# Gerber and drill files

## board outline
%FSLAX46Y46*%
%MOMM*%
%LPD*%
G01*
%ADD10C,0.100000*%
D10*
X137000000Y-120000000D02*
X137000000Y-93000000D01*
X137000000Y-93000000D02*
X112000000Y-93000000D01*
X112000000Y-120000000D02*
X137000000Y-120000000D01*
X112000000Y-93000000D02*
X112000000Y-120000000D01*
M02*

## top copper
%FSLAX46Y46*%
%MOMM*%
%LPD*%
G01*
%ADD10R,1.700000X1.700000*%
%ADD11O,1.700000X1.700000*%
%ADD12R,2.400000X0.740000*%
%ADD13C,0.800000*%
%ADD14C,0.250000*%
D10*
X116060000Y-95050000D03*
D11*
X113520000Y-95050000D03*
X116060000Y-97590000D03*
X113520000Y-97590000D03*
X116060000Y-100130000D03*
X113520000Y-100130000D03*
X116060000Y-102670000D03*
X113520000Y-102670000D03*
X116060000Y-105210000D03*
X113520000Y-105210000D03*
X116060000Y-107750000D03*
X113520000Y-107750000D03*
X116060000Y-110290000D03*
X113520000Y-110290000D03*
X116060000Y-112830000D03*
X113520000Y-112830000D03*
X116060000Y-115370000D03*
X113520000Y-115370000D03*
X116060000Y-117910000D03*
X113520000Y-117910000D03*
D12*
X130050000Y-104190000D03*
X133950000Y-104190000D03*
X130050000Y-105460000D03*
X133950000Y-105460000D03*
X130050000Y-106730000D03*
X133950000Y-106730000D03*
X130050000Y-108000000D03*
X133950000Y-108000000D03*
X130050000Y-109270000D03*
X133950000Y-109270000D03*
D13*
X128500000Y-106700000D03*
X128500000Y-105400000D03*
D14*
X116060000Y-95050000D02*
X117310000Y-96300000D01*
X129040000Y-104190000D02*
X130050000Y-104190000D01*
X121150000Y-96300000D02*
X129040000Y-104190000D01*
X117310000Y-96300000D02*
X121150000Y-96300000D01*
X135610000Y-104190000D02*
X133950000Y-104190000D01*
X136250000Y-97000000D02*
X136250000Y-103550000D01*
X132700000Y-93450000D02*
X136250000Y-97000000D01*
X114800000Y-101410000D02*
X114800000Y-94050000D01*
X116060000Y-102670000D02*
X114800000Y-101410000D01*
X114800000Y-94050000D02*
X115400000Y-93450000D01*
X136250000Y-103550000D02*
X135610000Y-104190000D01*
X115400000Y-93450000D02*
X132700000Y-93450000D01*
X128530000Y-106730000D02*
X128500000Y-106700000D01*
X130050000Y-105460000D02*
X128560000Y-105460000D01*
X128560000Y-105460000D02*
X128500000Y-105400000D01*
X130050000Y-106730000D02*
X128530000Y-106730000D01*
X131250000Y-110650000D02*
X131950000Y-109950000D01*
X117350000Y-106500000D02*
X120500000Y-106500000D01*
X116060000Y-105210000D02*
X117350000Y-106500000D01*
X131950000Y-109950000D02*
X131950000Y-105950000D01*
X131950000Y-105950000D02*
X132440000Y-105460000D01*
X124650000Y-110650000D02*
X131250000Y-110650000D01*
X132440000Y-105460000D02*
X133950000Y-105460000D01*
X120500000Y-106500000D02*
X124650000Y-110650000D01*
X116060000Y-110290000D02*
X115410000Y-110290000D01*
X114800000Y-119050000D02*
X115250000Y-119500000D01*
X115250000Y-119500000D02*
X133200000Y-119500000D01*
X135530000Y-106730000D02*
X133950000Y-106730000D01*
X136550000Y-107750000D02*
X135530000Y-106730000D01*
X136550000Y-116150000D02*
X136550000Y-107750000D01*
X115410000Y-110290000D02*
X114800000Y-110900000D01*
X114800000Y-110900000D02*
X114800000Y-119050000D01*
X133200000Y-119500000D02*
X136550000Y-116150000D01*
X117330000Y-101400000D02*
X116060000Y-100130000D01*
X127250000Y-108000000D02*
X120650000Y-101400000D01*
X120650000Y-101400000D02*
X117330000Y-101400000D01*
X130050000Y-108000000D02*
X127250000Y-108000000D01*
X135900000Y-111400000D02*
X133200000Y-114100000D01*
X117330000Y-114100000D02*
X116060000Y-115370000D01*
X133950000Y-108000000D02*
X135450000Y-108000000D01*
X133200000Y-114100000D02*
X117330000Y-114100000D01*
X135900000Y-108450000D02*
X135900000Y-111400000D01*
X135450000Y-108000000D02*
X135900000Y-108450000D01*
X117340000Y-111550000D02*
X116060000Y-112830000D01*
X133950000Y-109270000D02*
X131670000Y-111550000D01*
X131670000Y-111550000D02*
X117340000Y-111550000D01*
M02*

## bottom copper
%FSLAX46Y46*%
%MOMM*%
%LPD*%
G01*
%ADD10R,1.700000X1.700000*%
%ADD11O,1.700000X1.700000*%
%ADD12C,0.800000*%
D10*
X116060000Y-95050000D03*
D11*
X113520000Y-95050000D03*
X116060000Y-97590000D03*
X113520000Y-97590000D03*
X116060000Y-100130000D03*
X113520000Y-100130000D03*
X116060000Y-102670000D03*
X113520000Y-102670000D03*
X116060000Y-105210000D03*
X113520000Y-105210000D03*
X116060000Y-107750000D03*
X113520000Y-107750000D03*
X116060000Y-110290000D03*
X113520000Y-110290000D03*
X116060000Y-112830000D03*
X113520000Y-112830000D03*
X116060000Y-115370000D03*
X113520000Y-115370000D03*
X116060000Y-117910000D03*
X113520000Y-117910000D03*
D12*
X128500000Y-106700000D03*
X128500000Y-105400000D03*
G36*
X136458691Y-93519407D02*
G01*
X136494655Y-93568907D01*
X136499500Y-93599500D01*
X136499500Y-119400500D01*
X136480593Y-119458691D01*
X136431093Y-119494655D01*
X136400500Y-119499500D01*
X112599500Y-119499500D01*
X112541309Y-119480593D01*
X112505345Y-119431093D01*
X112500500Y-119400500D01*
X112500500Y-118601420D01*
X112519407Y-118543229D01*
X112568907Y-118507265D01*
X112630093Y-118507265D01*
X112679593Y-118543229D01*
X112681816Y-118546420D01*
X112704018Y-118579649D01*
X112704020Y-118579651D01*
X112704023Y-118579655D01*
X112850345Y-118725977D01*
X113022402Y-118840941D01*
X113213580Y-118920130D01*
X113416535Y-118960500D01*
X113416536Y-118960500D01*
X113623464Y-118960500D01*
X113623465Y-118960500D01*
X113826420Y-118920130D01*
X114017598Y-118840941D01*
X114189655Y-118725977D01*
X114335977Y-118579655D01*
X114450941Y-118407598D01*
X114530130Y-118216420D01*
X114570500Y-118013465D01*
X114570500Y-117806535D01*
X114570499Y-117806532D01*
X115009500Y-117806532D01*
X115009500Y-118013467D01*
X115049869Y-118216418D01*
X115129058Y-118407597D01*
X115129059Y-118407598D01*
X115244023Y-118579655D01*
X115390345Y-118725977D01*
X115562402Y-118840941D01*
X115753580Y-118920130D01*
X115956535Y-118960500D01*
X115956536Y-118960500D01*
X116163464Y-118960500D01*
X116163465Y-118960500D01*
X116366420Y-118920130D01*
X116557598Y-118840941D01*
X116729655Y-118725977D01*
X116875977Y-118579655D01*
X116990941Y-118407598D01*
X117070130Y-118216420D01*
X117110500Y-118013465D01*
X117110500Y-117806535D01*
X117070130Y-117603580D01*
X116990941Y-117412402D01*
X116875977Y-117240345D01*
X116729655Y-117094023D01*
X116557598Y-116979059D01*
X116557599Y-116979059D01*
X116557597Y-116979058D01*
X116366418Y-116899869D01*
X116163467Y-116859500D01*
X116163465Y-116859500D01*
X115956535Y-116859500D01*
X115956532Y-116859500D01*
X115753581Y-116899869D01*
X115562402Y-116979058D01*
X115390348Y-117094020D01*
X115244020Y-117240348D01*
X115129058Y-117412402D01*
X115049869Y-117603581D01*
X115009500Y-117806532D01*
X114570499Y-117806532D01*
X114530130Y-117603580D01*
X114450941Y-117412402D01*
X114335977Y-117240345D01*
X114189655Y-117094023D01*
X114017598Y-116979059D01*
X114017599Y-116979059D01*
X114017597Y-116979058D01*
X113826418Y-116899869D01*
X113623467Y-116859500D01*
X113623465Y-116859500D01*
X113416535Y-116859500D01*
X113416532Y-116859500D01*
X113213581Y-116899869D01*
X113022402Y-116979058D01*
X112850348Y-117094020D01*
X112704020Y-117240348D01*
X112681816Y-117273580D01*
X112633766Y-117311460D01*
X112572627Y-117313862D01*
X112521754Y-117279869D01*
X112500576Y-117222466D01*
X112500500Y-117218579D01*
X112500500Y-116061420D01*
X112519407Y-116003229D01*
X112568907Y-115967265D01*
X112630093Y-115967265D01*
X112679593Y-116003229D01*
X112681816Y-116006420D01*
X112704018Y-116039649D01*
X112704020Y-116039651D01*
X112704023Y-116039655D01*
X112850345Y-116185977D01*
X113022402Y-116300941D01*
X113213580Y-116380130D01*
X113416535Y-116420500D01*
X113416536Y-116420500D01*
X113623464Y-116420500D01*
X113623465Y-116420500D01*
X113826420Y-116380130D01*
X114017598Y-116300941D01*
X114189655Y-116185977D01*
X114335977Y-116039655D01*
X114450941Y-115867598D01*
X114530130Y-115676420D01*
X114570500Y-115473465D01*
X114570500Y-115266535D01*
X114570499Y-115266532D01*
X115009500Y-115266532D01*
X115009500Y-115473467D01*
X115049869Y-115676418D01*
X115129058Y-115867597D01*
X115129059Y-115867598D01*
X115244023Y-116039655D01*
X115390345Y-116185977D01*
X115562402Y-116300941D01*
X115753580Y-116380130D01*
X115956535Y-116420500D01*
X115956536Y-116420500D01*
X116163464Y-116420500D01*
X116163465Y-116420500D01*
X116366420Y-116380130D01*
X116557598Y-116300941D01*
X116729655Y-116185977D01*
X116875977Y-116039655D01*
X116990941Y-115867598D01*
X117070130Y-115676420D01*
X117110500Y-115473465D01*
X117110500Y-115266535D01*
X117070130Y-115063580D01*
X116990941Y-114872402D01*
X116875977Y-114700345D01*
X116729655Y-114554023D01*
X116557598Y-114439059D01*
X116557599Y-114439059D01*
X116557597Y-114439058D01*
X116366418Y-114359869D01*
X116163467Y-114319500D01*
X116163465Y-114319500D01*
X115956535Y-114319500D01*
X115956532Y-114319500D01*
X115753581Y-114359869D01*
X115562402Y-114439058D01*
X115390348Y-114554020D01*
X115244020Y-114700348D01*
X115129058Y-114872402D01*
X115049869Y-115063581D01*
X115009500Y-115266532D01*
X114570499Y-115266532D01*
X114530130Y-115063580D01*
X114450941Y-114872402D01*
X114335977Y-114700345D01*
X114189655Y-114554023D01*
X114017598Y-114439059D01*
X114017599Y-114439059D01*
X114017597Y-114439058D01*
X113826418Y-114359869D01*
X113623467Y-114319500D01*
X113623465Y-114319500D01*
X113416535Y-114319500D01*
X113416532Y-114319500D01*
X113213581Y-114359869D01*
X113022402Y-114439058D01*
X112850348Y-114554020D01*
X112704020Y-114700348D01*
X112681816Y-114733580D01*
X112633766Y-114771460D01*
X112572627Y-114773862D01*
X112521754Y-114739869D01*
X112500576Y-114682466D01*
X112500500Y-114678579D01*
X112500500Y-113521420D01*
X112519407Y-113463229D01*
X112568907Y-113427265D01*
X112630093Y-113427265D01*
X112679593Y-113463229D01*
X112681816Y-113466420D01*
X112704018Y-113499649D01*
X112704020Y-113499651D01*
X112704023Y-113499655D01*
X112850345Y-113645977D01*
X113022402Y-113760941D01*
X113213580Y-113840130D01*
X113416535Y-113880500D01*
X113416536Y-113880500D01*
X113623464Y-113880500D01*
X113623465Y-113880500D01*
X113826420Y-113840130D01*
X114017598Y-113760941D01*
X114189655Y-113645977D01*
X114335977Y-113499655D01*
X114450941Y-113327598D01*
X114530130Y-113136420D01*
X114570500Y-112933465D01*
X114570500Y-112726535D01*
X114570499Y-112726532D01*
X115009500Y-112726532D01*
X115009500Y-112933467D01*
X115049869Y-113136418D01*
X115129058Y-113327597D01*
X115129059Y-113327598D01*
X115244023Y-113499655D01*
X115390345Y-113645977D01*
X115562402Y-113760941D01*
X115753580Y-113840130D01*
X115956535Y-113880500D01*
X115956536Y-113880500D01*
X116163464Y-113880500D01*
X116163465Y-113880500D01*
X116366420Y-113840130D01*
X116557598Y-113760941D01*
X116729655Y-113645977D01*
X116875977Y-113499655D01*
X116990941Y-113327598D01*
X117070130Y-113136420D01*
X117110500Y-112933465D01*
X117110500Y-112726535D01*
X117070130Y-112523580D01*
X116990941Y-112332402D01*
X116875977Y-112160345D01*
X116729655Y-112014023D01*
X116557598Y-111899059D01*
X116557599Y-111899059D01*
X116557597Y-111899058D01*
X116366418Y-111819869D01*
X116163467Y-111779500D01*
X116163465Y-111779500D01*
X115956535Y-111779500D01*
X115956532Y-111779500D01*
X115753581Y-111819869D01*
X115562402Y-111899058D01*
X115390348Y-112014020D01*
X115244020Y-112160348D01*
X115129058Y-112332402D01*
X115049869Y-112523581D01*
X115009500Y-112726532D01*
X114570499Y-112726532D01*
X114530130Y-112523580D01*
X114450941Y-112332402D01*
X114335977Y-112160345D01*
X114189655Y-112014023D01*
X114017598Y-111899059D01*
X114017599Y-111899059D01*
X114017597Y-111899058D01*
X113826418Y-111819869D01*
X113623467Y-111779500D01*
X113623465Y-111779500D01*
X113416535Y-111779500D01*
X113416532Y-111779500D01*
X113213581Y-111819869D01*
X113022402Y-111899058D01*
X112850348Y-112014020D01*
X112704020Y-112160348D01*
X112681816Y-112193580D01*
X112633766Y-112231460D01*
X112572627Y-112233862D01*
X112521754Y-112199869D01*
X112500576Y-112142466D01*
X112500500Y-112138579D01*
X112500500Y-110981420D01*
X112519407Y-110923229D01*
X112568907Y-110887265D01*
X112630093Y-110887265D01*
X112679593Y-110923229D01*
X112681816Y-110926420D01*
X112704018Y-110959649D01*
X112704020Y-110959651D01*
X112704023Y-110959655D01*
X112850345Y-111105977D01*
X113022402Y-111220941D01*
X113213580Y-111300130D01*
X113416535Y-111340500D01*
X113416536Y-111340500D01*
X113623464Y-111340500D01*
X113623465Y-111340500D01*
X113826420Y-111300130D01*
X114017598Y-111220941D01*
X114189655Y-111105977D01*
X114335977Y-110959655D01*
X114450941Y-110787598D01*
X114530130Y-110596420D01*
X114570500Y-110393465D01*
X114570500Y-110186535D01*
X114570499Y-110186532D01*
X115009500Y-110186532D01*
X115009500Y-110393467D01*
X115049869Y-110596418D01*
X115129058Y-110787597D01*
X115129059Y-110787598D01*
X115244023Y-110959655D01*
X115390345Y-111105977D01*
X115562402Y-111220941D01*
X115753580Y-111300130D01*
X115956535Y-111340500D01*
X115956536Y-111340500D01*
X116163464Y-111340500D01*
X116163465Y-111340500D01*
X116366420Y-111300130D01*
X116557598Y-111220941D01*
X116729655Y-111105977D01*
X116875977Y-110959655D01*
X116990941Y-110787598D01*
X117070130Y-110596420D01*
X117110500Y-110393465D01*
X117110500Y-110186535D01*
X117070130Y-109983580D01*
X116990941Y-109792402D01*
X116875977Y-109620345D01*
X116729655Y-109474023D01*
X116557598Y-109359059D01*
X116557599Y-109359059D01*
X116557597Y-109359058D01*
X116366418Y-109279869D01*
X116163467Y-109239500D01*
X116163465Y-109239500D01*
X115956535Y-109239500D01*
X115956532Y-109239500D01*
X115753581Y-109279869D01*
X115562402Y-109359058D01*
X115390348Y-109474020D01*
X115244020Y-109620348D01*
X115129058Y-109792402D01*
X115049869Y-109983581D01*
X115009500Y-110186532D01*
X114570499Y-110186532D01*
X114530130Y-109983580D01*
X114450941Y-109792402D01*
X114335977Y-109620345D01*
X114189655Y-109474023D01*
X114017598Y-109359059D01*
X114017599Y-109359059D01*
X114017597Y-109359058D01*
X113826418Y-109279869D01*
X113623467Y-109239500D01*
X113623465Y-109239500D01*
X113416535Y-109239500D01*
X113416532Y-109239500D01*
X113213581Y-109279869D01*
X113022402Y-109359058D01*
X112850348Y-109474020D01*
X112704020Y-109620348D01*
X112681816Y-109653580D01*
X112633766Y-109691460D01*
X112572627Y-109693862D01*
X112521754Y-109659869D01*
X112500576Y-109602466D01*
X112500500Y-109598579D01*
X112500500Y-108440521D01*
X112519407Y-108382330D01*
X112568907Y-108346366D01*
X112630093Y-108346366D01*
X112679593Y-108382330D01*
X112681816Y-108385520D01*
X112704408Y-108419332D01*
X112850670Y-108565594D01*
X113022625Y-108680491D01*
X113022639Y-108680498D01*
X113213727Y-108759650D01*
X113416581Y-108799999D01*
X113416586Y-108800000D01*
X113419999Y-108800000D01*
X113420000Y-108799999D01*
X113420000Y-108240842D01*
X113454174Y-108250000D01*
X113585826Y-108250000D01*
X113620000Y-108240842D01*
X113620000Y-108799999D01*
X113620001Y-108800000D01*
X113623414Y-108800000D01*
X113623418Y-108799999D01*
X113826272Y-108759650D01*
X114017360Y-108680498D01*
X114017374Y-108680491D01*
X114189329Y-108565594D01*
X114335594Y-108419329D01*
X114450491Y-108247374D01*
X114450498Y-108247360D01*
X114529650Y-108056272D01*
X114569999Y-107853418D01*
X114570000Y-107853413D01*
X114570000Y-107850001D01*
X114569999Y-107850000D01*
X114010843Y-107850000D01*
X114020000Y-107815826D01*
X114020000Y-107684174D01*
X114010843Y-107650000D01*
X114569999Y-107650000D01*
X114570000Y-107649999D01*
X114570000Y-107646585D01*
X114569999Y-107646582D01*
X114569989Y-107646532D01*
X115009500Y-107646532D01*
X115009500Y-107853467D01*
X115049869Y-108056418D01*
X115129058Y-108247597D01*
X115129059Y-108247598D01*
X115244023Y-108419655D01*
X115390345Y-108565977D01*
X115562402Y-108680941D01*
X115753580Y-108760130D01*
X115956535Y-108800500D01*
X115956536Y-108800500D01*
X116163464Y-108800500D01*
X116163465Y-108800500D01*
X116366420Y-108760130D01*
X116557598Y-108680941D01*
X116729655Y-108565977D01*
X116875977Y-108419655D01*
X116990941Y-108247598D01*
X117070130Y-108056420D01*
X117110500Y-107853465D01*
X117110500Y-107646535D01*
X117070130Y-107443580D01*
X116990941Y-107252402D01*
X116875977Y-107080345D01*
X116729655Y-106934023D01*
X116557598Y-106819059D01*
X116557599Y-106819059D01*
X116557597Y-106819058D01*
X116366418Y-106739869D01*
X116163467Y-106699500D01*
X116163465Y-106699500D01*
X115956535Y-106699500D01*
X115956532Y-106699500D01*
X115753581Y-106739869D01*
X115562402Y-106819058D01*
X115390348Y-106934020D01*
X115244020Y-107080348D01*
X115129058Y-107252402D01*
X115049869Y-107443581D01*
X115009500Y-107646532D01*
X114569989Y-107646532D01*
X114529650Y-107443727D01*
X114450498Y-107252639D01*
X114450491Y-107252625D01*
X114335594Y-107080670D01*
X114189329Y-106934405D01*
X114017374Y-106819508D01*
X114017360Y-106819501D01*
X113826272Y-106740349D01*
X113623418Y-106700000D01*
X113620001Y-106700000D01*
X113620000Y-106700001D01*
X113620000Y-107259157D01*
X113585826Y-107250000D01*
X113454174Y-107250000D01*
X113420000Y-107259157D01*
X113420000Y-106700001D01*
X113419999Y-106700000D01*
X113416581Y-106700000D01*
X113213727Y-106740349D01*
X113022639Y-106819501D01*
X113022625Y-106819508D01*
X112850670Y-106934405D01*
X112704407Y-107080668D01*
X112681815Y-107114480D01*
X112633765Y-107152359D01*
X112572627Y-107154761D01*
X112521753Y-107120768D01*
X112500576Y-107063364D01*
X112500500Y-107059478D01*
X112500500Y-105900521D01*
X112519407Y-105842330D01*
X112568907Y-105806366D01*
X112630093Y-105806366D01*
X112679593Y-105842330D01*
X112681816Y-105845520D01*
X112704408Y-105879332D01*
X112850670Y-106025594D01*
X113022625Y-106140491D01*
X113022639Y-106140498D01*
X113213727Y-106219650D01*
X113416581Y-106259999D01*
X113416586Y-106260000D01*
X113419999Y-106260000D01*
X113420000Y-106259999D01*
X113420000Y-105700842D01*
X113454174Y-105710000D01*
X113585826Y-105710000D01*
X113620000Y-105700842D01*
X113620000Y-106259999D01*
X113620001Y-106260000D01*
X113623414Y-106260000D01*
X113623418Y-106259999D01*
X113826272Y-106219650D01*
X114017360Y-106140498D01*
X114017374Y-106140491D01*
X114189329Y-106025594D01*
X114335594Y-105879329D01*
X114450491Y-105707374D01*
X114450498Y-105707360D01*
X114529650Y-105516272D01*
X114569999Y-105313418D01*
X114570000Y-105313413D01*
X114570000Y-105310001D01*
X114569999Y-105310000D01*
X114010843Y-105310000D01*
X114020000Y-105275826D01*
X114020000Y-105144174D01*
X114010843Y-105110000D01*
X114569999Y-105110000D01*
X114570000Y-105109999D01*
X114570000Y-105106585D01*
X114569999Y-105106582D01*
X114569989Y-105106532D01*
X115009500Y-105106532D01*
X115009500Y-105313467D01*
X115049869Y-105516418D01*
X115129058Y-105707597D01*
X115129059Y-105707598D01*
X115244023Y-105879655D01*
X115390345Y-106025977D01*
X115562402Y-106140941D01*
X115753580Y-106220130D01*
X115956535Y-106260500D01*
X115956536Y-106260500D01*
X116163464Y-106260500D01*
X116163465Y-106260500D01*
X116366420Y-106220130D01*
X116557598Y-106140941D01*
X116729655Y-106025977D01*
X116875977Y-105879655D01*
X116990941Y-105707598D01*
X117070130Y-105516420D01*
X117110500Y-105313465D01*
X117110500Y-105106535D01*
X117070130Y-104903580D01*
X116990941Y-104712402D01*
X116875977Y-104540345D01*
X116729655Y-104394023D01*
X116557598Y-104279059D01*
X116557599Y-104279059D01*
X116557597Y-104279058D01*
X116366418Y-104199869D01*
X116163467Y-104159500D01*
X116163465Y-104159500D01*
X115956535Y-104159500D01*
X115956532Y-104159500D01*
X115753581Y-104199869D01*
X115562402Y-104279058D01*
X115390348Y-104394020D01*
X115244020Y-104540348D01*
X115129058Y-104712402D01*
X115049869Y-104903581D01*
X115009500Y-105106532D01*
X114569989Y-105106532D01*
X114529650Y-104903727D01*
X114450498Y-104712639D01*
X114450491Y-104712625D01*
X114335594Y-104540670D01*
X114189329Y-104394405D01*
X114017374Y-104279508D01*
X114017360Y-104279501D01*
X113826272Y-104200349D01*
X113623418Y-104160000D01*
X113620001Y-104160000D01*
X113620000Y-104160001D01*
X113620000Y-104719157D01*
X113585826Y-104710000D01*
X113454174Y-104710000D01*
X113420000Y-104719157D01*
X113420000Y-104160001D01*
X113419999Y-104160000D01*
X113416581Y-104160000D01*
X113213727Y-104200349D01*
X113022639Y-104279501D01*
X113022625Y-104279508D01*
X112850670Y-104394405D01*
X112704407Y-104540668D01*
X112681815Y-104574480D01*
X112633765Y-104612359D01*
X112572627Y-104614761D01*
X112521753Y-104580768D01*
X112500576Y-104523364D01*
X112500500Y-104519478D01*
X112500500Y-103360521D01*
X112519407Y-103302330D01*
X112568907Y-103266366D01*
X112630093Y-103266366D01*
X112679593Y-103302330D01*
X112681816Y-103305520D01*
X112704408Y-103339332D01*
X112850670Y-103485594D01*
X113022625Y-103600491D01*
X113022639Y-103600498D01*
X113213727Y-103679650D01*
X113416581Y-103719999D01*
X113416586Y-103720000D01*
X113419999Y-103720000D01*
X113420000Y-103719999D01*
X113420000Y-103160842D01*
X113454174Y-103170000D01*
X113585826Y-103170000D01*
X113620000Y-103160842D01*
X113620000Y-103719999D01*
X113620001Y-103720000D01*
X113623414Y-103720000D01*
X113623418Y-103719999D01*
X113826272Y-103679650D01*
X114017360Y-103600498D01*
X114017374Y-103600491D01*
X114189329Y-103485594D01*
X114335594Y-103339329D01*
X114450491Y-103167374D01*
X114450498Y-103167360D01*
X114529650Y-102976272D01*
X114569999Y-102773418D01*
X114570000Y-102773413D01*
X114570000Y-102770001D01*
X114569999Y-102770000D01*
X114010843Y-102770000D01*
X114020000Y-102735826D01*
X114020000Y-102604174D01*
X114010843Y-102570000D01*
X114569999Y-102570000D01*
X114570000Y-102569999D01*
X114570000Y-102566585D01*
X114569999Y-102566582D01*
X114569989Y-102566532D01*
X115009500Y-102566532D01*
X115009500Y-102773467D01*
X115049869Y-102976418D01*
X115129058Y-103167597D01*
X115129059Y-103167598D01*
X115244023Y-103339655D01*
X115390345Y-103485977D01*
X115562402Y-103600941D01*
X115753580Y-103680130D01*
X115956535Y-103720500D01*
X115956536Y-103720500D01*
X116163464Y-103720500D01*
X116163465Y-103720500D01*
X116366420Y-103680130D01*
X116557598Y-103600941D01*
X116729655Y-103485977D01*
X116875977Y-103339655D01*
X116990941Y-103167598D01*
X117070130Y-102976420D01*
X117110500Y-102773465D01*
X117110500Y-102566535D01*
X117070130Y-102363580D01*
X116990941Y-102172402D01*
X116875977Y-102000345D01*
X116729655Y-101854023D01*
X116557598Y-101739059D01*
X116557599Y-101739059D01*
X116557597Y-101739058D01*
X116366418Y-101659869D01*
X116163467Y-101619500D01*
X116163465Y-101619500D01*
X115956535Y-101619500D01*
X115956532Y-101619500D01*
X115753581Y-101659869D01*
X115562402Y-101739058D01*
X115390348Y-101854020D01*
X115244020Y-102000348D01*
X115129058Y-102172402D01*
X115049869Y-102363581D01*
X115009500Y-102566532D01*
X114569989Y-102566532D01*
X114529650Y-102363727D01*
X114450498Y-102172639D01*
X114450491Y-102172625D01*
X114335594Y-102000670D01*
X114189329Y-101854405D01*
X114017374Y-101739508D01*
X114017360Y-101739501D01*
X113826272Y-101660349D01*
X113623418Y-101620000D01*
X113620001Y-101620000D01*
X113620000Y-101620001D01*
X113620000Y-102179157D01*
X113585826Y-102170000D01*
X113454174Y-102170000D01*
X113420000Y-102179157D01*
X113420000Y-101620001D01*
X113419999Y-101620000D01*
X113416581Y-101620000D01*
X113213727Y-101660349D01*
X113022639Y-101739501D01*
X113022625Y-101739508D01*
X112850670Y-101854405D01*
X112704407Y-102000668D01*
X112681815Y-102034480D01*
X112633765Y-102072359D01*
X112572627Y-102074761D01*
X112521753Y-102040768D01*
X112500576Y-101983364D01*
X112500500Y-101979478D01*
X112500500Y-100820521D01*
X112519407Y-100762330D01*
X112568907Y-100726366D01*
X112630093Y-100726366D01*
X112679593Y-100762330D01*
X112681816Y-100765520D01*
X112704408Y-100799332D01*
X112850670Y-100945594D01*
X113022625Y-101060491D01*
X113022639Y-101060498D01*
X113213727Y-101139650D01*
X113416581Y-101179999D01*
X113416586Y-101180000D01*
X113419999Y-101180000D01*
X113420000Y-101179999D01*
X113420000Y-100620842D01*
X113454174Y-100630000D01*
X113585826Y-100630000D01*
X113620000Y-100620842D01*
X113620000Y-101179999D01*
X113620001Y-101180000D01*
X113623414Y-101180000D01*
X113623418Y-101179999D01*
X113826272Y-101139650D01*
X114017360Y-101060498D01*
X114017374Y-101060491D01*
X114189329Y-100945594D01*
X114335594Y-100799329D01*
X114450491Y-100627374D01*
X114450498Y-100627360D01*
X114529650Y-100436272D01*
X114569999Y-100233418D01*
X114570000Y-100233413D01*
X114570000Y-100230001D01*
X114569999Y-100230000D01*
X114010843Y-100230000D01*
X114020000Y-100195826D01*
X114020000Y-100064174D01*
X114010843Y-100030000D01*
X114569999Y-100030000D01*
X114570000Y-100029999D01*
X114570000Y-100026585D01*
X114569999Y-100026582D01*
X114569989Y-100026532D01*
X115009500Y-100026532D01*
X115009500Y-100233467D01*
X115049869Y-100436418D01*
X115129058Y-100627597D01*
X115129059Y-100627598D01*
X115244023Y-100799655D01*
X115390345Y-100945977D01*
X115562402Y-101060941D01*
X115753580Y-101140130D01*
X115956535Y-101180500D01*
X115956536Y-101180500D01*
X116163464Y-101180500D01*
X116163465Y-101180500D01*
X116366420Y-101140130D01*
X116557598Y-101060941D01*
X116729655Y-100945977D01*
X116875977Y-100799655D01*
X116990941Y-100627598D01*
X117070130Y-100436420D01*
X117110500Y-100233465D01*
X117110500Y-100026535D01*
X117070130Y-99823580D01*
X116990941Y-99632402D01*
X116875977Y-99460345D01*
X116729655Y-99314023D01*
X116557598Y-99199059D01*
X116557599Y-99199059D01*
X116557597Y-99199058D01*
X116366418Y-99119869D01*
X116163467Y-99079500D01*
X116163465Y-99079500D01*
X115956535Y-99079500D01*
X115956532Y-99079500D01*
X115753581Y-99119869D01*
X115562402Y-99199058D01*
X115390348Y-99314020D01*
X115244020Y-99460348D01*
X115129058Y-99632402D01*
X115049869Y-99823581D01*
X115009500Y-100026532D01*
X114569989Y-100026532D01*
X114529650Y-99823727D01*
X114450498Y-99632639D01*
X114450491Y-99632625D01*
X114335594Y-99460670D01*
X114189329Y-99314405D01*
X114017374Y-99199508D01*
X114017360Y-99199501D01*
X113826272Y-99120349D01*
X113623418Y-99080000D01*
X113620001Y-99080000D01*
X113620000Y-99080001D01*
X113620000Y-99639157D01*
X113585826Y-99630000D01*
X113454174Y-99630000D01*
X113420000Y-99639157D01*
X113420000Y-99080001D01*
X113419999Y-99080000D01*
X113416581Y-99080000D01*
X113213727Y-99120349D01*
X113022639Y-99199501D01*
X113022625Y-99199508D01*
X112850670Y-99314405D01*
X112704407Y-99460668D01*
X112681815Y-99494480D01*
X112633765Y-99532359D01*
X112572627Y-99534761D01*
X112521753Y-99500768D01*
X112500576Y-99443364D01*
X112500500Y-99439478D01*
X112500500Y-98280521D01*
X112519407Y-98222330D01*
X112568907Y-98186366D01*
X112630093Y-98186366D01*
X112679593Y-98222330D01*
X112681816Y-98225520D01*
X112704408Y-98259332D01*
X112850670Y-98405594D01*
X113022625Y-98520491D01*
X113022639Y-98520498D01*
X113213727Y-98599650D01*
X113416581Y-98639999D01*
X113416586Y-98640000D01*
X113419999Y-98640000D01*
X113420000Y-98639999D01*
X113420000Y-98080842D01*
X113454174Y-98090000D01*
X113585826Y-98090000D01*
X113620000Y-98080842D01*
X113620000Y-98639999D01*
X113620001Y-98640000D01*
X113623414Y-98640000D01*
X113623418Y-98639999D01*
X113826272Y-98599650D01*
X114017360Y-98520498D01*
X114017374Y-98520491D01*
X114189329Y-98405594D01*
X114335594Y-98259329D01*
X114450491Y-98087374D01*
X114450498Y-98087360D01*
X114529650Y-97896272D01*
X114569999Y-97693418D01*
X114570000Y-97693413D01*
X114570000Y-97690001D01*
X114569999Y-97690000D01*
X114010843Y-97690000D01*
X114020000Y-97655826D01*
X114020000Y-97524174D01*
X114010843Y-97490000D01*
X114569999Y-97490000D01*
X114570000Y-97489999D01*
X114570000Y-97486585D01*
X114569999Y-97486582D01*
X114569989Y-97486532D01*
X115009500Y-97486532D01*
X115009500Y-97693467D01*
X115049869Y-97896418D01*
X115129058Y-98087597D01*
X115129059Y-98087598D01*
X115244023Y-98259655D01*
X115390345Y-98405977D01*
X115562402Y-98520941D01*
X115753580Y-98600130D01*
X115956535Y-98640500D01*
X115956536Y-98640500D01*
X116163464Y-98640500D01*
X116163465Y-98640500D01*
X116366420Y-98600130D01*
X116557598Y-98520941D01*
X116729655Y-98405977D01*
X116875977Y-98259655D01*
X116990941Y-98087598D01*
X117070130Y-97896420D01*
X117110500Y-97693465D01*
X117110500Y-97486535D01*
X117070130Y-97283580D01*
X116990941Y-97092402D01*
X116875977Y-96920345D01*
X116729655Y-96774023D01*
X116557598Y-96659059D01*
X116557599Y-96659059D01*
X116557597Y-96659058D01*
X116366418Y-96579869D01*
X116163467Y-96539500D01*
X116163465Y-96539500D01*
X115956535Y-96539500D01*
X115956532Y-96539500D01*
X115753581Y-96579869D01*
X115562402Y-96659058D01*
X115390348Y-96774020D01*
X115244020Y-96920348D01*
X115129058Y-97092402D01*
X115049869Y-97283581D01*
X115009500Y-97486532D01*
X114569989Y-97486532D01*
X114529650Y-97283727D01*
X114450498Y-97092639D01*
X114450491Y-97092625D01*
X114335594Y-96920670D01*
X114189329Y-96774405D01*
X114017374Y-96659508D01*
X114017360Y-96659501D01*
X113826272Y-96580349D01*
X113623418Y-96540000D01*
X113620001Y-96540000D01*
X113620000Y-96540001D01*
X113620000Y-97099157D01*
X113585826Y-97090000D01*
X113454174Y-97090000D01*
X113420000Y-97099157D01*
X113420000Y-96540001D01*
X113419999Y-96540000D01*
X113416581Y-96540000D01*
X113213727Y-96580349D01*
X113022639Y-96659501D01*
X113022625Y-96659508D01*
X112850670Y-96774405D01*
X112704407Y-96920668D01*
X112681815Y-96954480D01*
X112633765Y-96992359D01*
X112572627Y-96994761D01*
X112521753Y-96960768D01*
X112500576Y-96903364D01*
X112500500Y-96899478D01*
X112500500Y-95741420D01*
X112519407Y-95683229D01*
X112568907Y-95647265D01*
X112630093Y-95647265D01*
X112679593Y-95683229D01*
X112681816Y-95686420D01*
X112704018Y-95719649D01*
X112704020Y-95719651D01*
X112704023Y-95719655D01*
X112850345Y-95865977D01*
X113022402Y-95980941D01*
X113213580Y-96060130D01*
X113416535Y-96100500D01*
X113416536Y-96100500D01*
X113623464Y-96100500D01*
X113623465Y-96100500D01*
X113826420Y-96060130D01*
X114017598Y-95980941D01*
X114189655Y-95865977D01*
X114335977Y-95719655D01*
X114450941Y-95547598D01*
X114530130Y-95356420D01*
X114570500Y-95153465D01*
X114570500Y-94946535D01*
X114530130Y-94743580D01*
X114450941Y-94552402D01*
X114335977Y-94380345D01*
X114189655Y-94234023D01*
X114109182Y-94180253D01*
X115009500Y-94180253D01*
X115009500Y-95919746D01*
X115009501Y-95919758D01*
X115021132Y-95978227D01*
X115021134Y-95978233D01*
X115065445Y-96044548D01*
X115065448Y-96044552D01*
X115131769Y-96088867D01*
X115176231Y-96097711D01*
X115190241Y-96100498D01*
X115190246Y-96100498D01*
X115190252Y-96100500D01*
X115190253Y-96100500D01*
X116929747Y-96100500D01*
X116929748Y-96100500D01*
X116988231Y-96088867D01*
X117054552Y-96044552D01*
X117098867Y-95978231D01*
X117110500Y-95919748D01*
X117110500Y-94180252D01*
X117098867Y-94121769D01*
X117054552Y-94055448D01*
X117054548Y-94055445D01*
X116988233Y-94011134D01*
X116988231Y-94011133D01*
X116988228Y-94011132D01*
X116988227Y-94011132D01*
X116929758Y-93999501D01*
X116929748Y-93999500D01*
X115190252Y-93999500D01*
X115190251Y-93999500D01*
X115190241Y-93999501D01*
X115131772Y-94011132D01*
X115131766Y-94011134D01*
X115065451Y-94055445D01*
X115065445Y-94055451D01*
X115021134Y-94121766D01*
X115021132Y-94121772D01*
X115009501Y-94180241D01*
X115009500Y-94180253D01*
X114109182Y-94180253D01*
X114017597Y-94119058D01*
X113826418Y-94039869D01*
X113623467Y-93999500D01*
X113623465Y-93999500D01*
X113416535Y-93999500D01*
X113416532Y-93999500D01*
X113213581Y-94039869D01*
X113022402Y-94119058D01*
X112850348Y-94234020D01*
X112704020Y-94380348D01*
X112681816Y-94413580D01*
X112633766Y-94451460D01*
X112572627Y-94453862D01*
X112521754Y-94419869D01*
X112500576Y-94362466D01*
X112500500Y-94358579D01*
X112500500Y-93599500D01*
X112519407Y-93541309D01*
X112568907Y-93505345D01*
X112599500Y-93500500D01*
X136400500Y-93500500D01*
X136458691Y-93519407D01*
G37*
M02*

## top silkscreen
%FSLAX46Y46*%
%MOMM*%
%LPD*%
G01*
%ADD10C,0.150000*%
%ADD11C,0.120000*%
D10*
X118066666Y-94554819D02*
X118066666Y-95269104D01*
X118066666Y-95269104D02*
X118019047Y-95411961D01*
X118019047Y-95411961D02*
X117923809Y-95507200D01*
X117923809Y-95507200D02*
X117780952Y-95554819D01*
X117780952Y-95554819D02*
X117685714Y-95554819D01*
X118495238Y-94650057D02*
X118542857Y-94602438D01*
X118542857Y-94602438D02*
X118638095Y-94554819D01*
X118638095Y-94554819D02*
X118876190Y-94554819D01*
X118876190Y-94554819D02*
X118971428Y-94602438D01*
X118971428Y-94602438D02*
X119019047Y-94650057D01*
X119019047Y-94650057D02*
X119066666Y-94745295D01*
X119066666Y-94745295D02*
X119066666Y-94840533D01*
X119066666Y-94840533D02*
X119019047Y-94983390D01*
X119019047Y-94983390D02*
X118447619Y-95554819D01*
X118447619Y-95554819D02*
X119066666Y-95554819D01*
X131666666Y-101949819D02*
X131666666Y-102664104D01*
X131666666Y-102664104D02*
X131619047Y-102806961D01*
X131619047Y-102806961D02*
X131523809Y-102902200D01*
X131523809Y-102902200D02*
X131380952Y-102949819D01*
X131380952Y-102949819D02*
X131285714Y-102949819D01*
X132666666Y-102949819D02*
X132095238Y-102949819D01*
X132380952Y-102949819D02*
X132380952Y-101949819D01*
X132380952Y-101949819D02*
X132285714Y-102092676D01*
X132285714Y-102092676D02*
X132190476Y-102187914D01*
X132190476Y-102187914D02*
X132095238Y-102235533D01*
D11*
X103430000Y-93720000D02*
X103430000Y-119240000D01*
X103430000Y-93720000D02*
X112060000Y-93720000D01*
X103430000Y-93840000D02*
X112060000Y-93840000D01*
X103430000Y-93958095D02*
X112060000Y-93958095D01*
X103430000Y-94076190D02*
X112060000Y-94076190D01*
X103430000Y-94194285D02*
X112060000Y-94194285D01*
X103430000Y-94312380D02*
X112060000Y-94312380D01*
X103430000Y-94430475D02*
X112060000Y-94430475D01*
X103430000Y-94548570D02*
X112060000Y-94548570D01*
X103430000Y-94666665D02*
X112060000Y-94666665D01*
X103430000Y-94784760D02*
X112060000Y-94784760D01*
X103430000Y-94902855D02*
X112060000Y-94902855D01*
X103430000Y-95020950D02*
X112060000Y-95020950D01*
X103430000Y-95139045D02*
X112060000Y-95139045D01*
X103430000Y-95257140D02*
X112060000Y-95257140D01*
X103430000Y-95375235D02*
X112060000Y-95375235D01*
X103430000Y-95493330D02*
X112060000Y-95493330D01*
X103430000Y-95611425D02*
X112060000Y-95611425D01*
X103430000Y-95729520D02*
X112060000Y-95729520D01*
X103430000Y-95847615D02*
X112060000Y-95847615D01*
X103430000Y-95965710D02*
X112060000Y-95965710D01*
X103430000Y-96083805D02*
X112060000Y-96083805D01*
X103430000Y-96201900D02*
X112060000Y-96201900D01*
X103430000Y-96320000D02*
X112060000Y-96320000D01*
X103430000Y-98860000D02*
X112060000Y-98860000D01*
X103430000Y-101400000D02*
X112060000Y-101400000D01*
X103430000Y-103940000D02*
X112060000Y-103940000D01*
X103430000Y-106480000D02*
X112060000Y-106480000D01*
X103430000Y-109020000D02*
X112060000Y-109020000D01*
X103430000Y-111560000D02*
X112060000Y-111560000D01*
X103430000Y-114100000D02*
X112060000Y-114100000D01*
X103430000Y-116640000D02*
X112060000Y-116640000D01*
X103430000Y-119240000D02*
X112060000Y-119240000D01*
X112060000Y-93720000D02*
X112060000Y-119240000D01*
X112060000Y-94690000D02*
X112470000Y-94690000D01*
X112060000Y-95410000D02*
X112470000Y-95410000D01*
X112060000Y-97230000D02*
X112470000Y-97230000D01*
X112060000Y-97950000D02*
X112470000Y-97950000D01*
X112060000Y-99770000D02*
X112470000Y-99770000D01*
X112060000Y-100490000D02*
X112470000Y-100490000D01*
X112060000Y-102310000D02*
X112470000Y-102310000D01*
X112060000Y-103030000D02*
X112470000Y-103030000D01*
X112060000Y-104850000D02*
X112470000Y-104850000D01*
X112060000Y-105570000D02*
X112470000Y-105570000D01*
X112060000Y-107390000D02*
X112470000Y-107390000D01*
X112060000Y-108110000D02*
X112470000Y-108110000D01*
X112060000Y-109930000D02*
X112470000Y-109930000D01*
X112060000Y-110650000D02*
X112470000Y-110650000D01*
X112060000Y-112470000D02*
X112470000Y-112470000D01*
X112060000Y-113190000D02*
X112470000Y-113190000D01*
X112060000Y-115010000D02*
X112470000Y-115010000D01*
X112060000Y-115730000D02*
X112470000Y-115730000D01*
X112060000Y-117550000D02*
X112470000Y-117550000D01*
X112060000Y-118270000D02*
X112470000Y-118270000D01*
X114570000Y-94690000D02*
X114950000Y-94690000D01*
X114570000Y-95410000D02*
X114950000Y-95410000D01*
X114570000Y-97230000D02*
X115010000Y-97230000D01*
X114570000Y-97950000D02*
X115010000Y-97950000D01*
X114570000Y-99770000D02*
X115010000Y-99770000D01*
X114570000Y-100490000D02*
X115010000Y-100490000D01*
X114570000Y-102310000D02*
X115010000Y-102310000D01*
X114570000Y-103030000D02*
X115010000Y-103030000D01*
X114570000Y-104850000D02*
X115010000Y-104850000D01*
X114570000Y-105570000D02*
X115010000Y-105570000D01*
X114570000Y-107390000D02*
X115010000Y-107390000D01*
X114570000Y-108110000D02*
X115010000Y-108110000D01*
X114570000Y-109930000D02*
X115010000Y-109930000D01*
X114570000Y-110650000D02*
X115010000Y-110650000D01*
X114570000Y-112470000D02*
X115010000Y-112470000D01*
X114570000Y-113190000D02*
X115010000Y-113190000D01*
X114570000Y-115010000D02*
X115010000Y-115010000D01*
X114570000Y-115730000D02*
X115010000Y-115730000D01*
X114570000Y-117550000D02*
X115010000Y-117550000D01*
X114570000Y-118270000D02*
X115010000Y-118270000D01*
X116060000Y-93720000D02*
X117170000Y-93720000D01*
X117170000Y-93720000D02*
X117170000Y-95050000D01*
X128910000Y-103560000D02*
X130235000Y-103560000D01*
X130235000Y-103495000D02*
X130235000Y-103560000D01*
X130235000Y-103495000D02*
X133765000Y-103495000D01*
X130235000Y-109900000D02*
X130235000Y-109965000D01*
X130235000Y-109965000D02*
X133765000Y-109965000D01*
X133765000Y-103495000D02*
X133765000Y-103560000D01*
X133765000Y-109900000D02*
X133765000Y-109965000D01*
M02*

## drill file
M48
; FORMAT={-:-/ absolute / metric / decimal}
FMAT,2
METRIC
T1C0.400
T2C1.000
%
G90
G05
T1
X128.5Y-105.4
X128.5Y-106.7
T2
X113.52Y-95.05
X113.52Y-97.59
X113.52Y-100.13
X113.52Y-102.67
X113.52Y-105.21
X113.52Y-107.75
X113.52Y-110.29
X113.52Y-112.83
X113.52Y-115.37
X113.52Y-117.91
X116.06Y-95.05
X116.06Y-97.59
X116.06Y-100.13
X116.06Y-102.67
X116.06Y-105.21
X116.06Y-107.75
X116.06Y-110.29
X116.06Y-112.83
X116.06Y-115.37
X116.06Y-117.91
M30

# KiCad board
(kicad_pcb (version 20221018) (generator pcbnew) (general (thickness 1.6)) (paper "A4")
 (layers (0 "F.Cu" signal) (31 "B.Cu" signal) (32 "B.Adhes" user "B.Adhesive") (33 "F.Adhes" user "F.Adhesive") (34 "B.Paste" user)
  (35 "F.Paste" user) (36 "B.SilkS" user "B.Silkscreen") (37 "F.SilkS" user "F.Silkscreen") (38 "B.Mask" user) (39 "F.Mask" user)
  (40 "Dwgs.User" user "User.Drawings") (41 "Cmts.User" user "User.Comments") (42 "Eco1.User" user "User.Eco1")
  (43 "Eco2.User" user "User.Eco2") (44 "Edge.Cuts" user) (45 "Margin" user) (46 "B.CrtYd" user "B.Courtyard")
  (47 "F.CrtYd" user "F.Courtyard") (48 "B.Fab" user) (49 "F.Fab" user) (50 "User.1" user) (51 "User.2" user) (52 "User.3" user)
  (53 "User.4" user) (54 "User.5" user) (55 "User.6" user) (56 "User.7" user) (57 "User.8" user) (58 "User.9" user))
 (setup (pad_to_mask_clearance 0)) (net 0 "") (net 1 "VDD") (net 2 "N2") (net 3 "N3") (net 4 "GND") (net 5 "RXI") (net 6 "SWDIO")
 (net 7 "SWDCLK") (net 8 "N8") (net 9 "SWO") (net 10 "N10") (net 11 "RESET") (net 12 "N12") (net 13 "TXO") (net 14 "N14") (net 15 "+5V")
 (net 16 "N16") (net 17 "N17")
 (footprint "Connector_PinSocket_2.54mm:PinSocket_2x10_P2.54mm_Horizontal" (layer "F.Cu") (at 116.06 95.05)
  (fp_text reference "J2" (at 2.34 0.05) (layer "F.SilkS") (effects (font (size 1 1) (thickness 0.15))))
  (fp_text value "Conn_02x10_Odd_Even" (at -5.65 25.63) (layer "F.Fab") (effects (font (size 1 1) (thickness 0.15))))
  (fp_line (start -12.63 -1.33) (end -12.63 24.19) (stroke (width 0.12) (type solid)) (layer "F.SilkS"))
  (fp_line (start -12.63 -1.33) (end -4 -1.33) (stroke (width 0.12) (type solid)) (layer "F.SilkS"))
  (fp_line (start -12.63 -1.21) (end -4 -1.21) (stroke (width 0.12) (type solid)) (layer "F.SilkS"))
  (fp_line (start -12.63 -1.091905) (end -4 -1.091905) (stroke (width 0.12) (type solid)) (layer "F.SilkS"))
  (fp_line (start -12.63 -0.97381) (end -4 -0.97381) (stroke (width 0.12) (type solid)) (layer "F.SilkS"))
  (fp_line (start -12.63 -0.855715) (end -4 -0.855715) (stroke (width 0.12) (type solid)) (layer "F.SilkS"))
  (fp_line (start -12.63 -0.73762) (end -4 -0.73762) (stroke (width 0.12) (type solid)) (layer "F.SilkS"))
  (fp_line (start -12.63 -0.619525) (end -4 -0.619525) (stroke (width 0.12) (type solid)) (layer "F.SilkS"))
  (fp_line (start -12.63 -0.50143) (end -4 -0.50143) (stroke (width 0.12) (type solid)) (layer "F.SilkS"))
  (fp_line (start -12.63 -0.383335) (end -4 -0.383335) (stroke (width 0.12) (type solid)) (layer "F.SilkS"))
  (fp_line (start -12.63 -0.26524) (end -4 -0.26524) (stroke (width 0.12) (type solid)) (layer "F.SilkS"))
  (fp_line (start -12.63 -0.147145) (end -4 -0.147145) (stroke (width 0.12) (type solid)) (layer "F.SilkS"))
  (fp_line (start -12.63 -0.02905) (end -4 -0.02905) (stroke (width 0.12) (type solid)) (layer "F.SilkS"))
  (fp_line (start -12.63 0.089045) (end -4 0.089045) (stroke (width 0.12) (type solid)) (layer "F.SilkS"))
  (fp_line (start -12.63 0.20714) (end -4 0.20714) (stroke (width 0.12) (type solid)) (layer "F.SilkS"))
  (fp_line (start -12.63 0.325235) (end -4 0.325235) (stroke (width 0.12) (type solid)) (layer "F.SilkS"))
  (fp_line (start -12.63 0.44333) (end -4 0.44333) (stroke (width 0.12) (type solid)) (layer "F.SilkS"))
  (fp_line (start -12.63 0.561425) (end -4 0.561425) (stroke (width 0.12) (type solid)) (layer "F.SilkS"))
  (fp_line (start -12.63 0.67952) (end -4 0.67952) (stroke (width 0.12) (type solid)) (layer "F.SilkS"))
  (fp_line (start -12.63 0.797615) (end -4 0.797615) (stroke (width 0.12) (type solid)) (layer "F.SilkS"))
  (fp_line (start -12.63 0.91571) (end -4 0.91571) (stroke (width 0.12) (type solid)) (layer "F.SilkS"))
  (fp_line (start -12.63 1.033805) (end -4 1.033805) (stroke (width 0.12) (type solid)) (layer "F.SilkS"))
  (fp_line (start -12.63 1.1519) (end -4 1.1519) (stroke (width 0.12) (type solid)) (layer "F.SilkS"))
  (fp_line (start -12.63 1.27) (end -4 1.27) (stroke (width 0.12) (type solid)) (layer "F.SilkS"))
  (fp_line (start -12.63 3.81) (end -4 3.81) (stroke (width 0.12) (type solid)) (layer "F.SilkS"))
  (fp_line (start -12.63 6.35) (end -4 6.35) (stroke (width 0.12) (type solid)) (layer "F.SilkS"))
  (fp_line (start -12.63 8.89) (end -4 8.89) (stroke (width 0.12) (type solid)) (layer "F.SilkS"))
  (fp_line (start -12.63 11.43) (end -4 11.43) (stroke (width 0.12) (type solid)) (layer "F.SilkS"))
  (fp_line (start -12.63 13.97) (end -4 13.97) (stroke (width 0.12) (type solid)) (layer "F.SilkS"))
  (fp_line (start -12.63 16.51) (end -4 16.51) (stroke (width 0.12) (type solid)) (layer "F.SilkS"))
  (fp_line (start -12.63 19.05) (end -4 19.05) (stroke (width 0.12) (type solid)) (layer "F.SilkS"))
  (fp_line (start -12.63 21.59) (end -4 21.59) (stroke (width 0.12) (type solid)) (layer "F.SilkS"))
  (fp_line (start -12.63 24.19) (end -4 24.19) (stroke (width 0.12) (type solid)) (layer "F.SilkS"))
  (fp_line (start -4 -1.33) (end -4 24.19) (stroke (width 0.12) (type solid)) (layer "F.SilkS"))
  (fp_line (start -4 -0.36) (end -3.59 -0.36) (stroke (width 0.12) (type solid)) (layer "F.SilkS"))
  (fp_line (start -4 0.36) (end -3.59 0.36) (stroke (width 0.12) (type solid)) (layer "F.SilkS"))
  (fp_line (start -4 2.18) (end -3.59 2.18) (stroke (width 0.12) (type solid)) (layer "F.SilkS"))
  (fp_line (start -4 2.9) (end -3.59 2.9) (stroke (width 0.12) (type solid)) (layer "F.SilkS"))
  (fp_line (start -4 4.72) (end -3.59 4.72) (stroke (width 0.12) (type solid)) (layer "F.SilkS"))
  (fp_line (start -4 5.44) (end -3.59 5.44) (stroke (width 0.12) (type solid)) (layer "F.SilkS"))
  (fp_line (start -4 7.26) (end -3.59 7.26) (stroke (width 0.12) (type solid)) (layer "F.SilkS"))
  (fp_line (start -4 7.98) (end -3.59 7.98) (stroke (width 0.12) (type solid)) (layer "F.SilkS"))
  (fp_line (start -4 9.8) (end -3.59 9.8) (stroke (width 0.12) (type solid)) (layer "F.SilkS"))
  (fp_line (start -4 10.52) (end -3.59 10.52) (stroke (width 0.12) (type solid)) (layer "F.SilkS"))
  (fp_line (start -4 12.34) (end -3.59 12.34) (stroke (width 0.12) (type solid)) (layer "F.SilkS"))
  (fp_line (start -4 13.06) (end -3.59 13.06) (stroke (width 0.12) (type solid)) (layer "F.SilkS"))
  (fp_line (start -4 14.88) (end -3.59 14.88) (stroke (width 0.12) (type solid)) (layer "F.SilkS"))
  (fp_line (start -4 15.6) (end -3.59 15.6) (stroke (width 0.12) (type solid)) (layer "F.SilkS"))
  (fp_line (start -4 17.42) (end -3.59 17.42) (stroke (width 0.12) (type solid)) (layer "F.SilkS"))
  (fp_line (start -4 18.14) (end -3.59 18.14) (stroke (width 0.12) (type solid)) (layer "F.SilkS"))
  (fp_line (start -4 19.96) (end -3.59 19.96) (stroke (width 0.12) (type solid)) (layer "F.SilkS"))
  (fp_line (start -4 20.68) (end -3.59 20.68) (stroke (width 0.12) (type solid)) (layer "F.SilkS"))
  (fp_line (start -4 22.5) (end -3.59 22.5) (stroke (width 0.12) (type solid)) (layer "F.SilkS"))
  (fp_line (start -4 23.22) (end -3.59 23.22) (stroke (width 0.12) (type solid)) (layer "F.SilkS"))
  (fp_line (start -1.49 -0.36) (end -1.11 -0.36) (stroke (width 0.12) (type solid)) (layer "F.SilkS"))
  (fp_line (start -1.49 0.36) (end -1.11 0.36) (stroke (width 0.12) (type solid)) (layer "F.SilkS"))
  (fp_line (start -1.49 2.18) (end -1.05 2.18) (stroke (width 0.12) (type solid)) (layer "F.SilkS"))
  (fp_line (start -1.49 2.9) (end -1.05 2.9) (stroke (width 0.12) (type solid)) (layer "F.SilkS"))
  (fp_line (start -1.49 4.72) (end -1.05 4.72) (stroke (width 0.12) (type solid)) (layer "F.SilkS"))
  (fp_line (start -1.49 5.44) (end -1.05 5.44) (stroke (width 0.12) (type solid)) (layer "F.SilkS"))
  (fp_line (start -1.49 7.26) (end -1.05 7.26) (stroke (width 0.12) (type solid)) (layer "F.SilkS"))
  (fp_line (start -1.49 7.98) (end -1.05 7.98) (stroke (width 0.12) (type solid)) (layer "F.SilkS"))
  (fp_line (start -1.49 9.8) (end -1.05 9.8) (stroke (width 0.12) (type solid)) (layer "F.SilkS"))
  (fp_line (start -1.49 10.52) (end -1.05 10.52) (stroke (width 0.12) (type solid)) (layer "F.SilkS"))
  (fp_line (start -1.49 12.34) (end -1.05 12.34) (stroke (width 0.12) (type solid)) (layer "F.SilkS"))
  (fp_line (start -1.49 13.06) (end -1.05 13.06) (stroke (width 0.12) (type solid)) (layer "F.SilkS"))
  (fp_line (start -1.49 14.88) (end -1.05 14.88) (stroke (width 0.12) (type solid)) (layer "F.SilkS"))
  (fp_line (start -1.49 15.6) (end -1.05 15.6) (stroke (width 0.12) (type solid)) (layer "F.SilkS"))
  (fp_line (start -1.49 17.42) (end -1.05 17.42) (stroke (width 0.12) (type solid)) (layer "F.SilkS"))
  (fp_line (start -1.49 18.14) (end -1.05 18.14) (stroke (width 0.12) (type solid)) (layer "F.SilkS"))
  (fp_line (start -1.49 19.96) (end -1.05 19.96) (stroke (width 0.12) (type solid)) (layer "F.SilkS"))
  (fp_line (start -1.49 20.68) (end -1.05 20.68) (stroke (width 0.12) (type solid)) (layer "F.SilkS"))
  (fp_line (start -1.49 22.5) (end -1.05 22.5) (stroke (width 0.12) (type solid)) (layer "F.SilkS"))
  (fp_line (start -1.49 23.22) (end -1.05 23.22) (stroke (width 0.12) (type solid)) (layer "F.SilkS"))
  (fp_line (start 0 -1.33) (end 1.11 -1.33) (stroke (width 0.12) (type solid)) (layer "F.SilkS"))
  (fp_line (start 1.11 -1.33) (end 1.11 0) (stroke (width 0.12) (type solid)) (layer "F.SilkS"))
  (pad "1" thru_hole rect (at 0 0) (size 1.7 1.7) (drill 1) (layers "*.Cu" "*.Mask") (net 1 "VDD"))
  (pad "2" thru_hole oval (at -2.54 0) (size 1.7 1.7) (drill 1) (layers "*.Cu" "*.Mask") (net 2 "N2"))
  (pad "3" thru_hole oval (at 0 2.54) (size 1.7 1.7) (drill 1) (layers "*.Cu" "*.Mask") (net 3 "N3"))
  (pad "4" thru_hole oval (at -2.54 2.54) (size 1.7 1.7) (drill 1) (layers "*.Cu" "*.Mask") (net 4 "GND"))
  (pad "5" thru_hole oval (at 0 5.08) (size 1.7 1.7) (drill 1) (layers "*.Cu" "*.Mask") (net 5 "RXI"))
  (pad "6" thru_hole oval (at -2.54 5.08) (size 1.7 1.7) (drill 1) (layers "*.Cu" "*.Mask") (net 4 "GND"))
  (pad "7" thru_hole oval (at 0 7.62) (size 1.7 1.7) (drill 1) (layers "*.Cu" "*.Mask") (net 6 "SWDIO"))
  (pad "8" thru_hole oval (at -2.54 7.62) (size 1.7 1.7) (drill 1) (layers "*.Cu" "*.Mask") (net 4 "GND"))
  (pad "9" thru_hole oval (at 0 10.16) (size 1.7 1.7) (drill 1) (layers "*.Cu" "*.Mask") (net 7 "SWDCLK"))
  (pad "10" thru_hole oval (at -2.54 10.16) (size 1.7 1.7) (drill 1) (layers "*.Cu" "*.Mask") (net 4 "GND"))
  (pad "11" thru_hole oval (at 0 12.7) (size 1.7 1.7) (drill 1) (layers "*.Cu" "*.Mask") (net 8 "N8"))
  (pad "12" thru_hole oval (at -2.54 12.7) (size 1.7 1.7) (drill 1) (layers "*.Cu" "*.Mask") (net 4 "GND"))
  (pad "13" thru_hole oval (at 0 15.24) (size 1.7 1.7) (drill 1) (layers "*.Cu" "*.Mask") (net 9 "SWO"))
  (pad "14" thru_hole oval (at -2.54 15.24) (size 1.7 1.7) (drill 1) (layers "*.Cu" "*.Mask") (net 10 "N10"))
  (pad "15" thru_hole oval (at 0 17.78) (size 1.7 1.7) (drill 1) (layers "*.Cu" "*.Mask") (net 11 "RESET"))
  (pad "16" thru_hole oval (at -2.54 17.78) (size 1.7 1.7) (drill 1) (layers "*.Cu" "*.Mask") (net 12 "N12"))
  (pad "17" thru_hole oval (at 0 20.32) (size 1.7 1.7) (drill 1) (layers "*.Cu" "*.Mask") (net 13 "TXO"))
  (pad "18" thru_hole oval (at -2.54 20.32) (size 1.7 1.7) (drill 1) (layers "*.Cu" "*.Mask") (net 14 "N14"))
  (pad "19" thru_hole oval (at 0 22.86) (size 1.7 1.7) (drill 1) (layers "*.Cu" "*.Mask") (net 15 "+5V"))
  (pad "20" thru_hole oval (at -2.54 22.86) (size 1.7 1.7) (drill 1) (layers "*.Cu" "*.Mask") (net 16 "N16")))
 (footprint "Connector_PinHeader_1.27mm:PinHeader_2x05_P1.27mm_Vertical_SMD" (layer "F.Cu") (at 132 106.73)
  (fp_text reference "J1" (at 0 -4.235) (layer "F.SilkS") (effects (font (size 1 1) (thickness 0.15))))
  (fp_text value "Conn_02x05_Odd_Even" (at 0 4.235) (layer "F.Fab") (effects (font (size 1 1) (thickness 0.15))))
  (fp_line (start -3.09 -3.17) (end -1.765 -3.17) (stroke (width 0.12) (type solid)) (layer "F.SilkS"))
  (fp_line (start -1.765 -3.235) (end -1.765 -3.17) (stroke (width 0.12) (type solid)) (layer "F.SilkS"))
  (fp_line (start -1.765 -3.235) (end 1.765 -3.235) (stroke (width 0.12) (type solid)) (layer "F.SilkS"))
  (fp_line (start -1.765 3.17) (end -1.765 3.235) (stroke (width 0.12) (type solid)) (layer "F.SilkS"))
  (fp_line (start -1.765 3.235) (end 1.765 3.235) (stroke (width 0.12) (type solid)) (layer "F.SilkS"))
  (fp_line (start 1.765 -3.235) (end 1.765 -3.17) (stroke (width 0.12) (type solid)) (layer "F.SilkS"))
  (fp_line (start 1.765 3.17) (end 1.765 3.235) (stroke (width 0.12) (type solid)) (layer "F.SilkS"))
  (pad "1" smd rect (at -1.95 -2.54) (size 2.4 0.74) (layers "F.Cu" "F.Paste" "F.Mask") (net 1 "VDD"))
  (pad "2" smd rect (at 1.95 -2.54) (size 2.4 0.74) (layers "F.Cu" "F.Paste" "F.Mask") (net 6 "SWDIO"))
  (pad "3" smd rect (at -1.95 -1.27) (size 2.4 0.74) (layers "F.Cu" "F.Paste" "F.Mask") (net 4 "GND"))
  (pad "4" smd rect (at 1.95 -1.27) (size 2.4 0.74) (layers "F.Cu" "F.Paste" "F.Mask") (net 7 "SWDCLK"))
  (pad "5" smd rect (at -1.95 0) (size 2.4 0.74) (layers "F.Cu" "F.Paste" "F.Mask") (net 4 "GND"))
  (pad "6" smd rect (at 1.95 0) (size 2.4 0.74) (layers "F.Cu" "F.Paste" "F.Mask") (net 9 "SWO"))
  (pad "7" smd rect (at -1.95 1.27) (size 2.4 0.74) (layers "F.Cu" "F.Paste" "F.Mask") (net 5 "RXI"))
  (pad "8" smd rect (at 1.95 1.27) (size 2.4 0.74) (layers "F.Cu" "F.Paste" "F.Mask") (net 13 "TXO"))
  (pad "9" smd rect (at -1.95 2.54) (size 2.4 0.74) (layers "F.Cu" "F.Paste" "F.Mask") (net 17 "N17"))
  (pad "10" smd rect (at 1.95 2.54) (size 2.4 0.74) (layers "F.Cu" "F.Paste" "F.Mask") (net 11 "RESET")))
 (gr_line (start 137 120) (end 137 93) (stroke (width 0.1) (type default)) (layer "Edge.Cuts"))
 (gr_line (start 137 93) (end 112 93) (stroke (width 0.1) (type default)) (layer "Edge.Cuts"))
 (gr_line (start 112 120) (end 137 120) (stroke (width 0.1) (type default)) (layer "Edge.Cuts"))
 (gr_line (start 112 93) (end 112 120) (stroke (width 0.1) (type default)) (layer "Edge.Cuts"))
 (segment (start 116.06 95.05) (end 117.31 96.3) (width 0.25) (layer "F.Cu") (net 1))
 (segment (start 129.04 104.19) (end 130.05 104.19) (width 0.25) (layer "F.Cu") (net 1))
 (segment (start 121.15 96.3) (end 129.04 104.19) (width 0.25) (layer "F.Cu") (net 1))
 (segment (start 117.31 96.3) (end 121.15 96.3) (width 0.25) (layer "F.Cu") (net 1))
 (segment (start 135.61 104.19) (end 133.95 104.19) (width 0.25) (layer "F.Cu") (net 6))
 (segment (start 136.25 97) (end 136.25 103.55) (width 0.25) (layer "F.Cu") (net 6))
 (segment (start 132.7 93.45) (end 136.25 97) (width 0.25) (layer "F.Cu") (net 6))
 (segment (start 114.8 101.41) (end 114.8 94.05) (width 0.25) (layer "F.Cu") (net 6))
 (segment (start 116.06 102.67) (end 114.8 101.41) (width 0.25) (layer "F.Cu") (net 6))
 (segment (start 114.8 94.05) (end 115.4 93.45) (width 0.25) (layer "F.Cu") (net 6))
 (segment (start 136.25 103.55) (end 135.61 104.19) (width 0.25) (layer "F.Cu") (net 6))
 (segment (start 115.4 93.45) (end 132.7 93.45) (width 0.25) (layer "F.Cu") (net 6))
 (segment (start 128.53 106.73) (end 128.5 106.7) (width 0.25) (layer "F.Cu") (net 4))
 (segment (start 130.05 105.46) (end 128.56 105.46) (width 0.25) (layer "F.Cu") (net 4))
 (segment (start 128.56 105.46) (end 128.5 105.4) (width 0.25) (layer "F.Cu") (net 4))
 (segment (start 130.05 106.73) (end 128.53 106.73) (width 0.25) (layer "F.Cu") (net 4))
 (via (at 128.5 106.7) (size 0.8) (drill 0.4) (layers "F.Cu" "B.Cu") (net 4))
 (via (at 128.5 105.4) (size 0.8) (drill 0.4) (layers "F.Cu" "B.Cu") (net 4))
 (segment (start 131.25 110.65) (end 131.95 109.95) (width 0.25) (layer "F.Cu") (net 7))
 (segment (start 117.35 106.5) (end 120.5 106.5) (width 0.25) (layer "F.Cu") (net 7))
 (segment (start 116.06 105.21) (end 117.35 106.5) (width 0.25) (layer "F.Cu") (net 7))
 (segment (start 131.95 109.95) (end 131.95 105.95) (width 0.25) (layer "F.Cu") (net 7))
 (segment (start 131.95 105.95) (end 132.44 105.46) (width 0.25) (layer "F.Cu") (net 7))
 (segment (start 124.65 110.65) (end 131.25 110.65) (width 0.25) (layer "F.Cu") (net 7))
 (segment (start 132.44 105.46) (end 133.95 105.46) (width 0.25) (layer "F.Cu") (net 7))
 (segment (start 120.5 106.5) (end 124.65 110.65) (width 0.25) (layer "F.Cu") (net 7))
 (segment (start 116.06 110.29) (end 115.41 110.29) (width 0.25) (layer "F.Cu") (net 9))
 (segment (start 114.8 119.05) (end 115.25 119.5) (width 0.25) (layer "F.Cu") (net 9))
 (segment (start 115.25 119.5) (end 133.2 119.5) (width 0.25) (layer "F.Cu") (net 9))
 (segment (start 135.53 106.73) (end 133.95 106.73) (width 0.25) (layer "F.Cu") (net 9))
 (segment (start 136.55 107.75) (end 135.53 106.73) (width 0.25) (layer "F.Cu") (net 9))
 (segment (start 136.55 116.15) (end 136.55 107.75) (width 0.25) (layer "F.Cu") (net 9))
 (segment (start 115.41 110.29) (end 114.8 110.9) (width 0.25) (layer "F.Cu") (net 9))
 (segment (start 114.8 110.9) (end 114.8 119.05) (width 0.25) (layer "F.Cu") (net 9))
 (segment (start 133.2 119.5) (end 136.55 116.15) (width 0.25) (layer "F.Cu") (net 9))
 (segment (start 117.33 101.4) (end 116.06 100.13) (width 0.25) (layer "F.Cu") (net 5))
 (segment (start 127.25 108) (end 120.65 101.4) (width 0.25) (layer "F.Cu") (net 5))
 (segment (start 120.65 101.4) (end 117.33 101.4) (width 0.25) (layer "F.Cu") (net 5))
 (segment (start 130.05 108) (end 127.25 108) (width 0.25) (layer "F.Cu") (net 5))
 (segment (start 135.9 111.4) (end 133.2 114.1) (width 0.25) (layer "F.Cu") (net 13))
 (segment (start 117.33 114.1) (end 116.06 115.37) (width 0.25) (layer "F.Cu") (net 13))
 (segment (start 133.95 108) (end 135.45 108) (width 0.25) (layer "F.Cu") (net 13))
 (segment (start 133.2 114.1) (end 117.33 114.1) (width 0.25) (layer "F.Cu") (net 13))
 (segment (start 135.9 108.45) (end 135.9 111.4) (width 0.25) (layer "F.Cu") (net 13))
 (segment (start 135.45 108) (end 135.9 108.45) (width 0.25) (layer "F.Cu") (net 13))
 (segment (start 117.34 111.55) (end 116.06 112.83) (width 0.25) (layer "F.Cu") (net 11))
 (segment (start 133.95 109.27) (end 131.67 111.55) (width 0.25) (layer "F.Cu") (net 11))
 (segment (start 131.67 111.55) (end 117.34 111.55) (width 0.25) (layer "F.Cu") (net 11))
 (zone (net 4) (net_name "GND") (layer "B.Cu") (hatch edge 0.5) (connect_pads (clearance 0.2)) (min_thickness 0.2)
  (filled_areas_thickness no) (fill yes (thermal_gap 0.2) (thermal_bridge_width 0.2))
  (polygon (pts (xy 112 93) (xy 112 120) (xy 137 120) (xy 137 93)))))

